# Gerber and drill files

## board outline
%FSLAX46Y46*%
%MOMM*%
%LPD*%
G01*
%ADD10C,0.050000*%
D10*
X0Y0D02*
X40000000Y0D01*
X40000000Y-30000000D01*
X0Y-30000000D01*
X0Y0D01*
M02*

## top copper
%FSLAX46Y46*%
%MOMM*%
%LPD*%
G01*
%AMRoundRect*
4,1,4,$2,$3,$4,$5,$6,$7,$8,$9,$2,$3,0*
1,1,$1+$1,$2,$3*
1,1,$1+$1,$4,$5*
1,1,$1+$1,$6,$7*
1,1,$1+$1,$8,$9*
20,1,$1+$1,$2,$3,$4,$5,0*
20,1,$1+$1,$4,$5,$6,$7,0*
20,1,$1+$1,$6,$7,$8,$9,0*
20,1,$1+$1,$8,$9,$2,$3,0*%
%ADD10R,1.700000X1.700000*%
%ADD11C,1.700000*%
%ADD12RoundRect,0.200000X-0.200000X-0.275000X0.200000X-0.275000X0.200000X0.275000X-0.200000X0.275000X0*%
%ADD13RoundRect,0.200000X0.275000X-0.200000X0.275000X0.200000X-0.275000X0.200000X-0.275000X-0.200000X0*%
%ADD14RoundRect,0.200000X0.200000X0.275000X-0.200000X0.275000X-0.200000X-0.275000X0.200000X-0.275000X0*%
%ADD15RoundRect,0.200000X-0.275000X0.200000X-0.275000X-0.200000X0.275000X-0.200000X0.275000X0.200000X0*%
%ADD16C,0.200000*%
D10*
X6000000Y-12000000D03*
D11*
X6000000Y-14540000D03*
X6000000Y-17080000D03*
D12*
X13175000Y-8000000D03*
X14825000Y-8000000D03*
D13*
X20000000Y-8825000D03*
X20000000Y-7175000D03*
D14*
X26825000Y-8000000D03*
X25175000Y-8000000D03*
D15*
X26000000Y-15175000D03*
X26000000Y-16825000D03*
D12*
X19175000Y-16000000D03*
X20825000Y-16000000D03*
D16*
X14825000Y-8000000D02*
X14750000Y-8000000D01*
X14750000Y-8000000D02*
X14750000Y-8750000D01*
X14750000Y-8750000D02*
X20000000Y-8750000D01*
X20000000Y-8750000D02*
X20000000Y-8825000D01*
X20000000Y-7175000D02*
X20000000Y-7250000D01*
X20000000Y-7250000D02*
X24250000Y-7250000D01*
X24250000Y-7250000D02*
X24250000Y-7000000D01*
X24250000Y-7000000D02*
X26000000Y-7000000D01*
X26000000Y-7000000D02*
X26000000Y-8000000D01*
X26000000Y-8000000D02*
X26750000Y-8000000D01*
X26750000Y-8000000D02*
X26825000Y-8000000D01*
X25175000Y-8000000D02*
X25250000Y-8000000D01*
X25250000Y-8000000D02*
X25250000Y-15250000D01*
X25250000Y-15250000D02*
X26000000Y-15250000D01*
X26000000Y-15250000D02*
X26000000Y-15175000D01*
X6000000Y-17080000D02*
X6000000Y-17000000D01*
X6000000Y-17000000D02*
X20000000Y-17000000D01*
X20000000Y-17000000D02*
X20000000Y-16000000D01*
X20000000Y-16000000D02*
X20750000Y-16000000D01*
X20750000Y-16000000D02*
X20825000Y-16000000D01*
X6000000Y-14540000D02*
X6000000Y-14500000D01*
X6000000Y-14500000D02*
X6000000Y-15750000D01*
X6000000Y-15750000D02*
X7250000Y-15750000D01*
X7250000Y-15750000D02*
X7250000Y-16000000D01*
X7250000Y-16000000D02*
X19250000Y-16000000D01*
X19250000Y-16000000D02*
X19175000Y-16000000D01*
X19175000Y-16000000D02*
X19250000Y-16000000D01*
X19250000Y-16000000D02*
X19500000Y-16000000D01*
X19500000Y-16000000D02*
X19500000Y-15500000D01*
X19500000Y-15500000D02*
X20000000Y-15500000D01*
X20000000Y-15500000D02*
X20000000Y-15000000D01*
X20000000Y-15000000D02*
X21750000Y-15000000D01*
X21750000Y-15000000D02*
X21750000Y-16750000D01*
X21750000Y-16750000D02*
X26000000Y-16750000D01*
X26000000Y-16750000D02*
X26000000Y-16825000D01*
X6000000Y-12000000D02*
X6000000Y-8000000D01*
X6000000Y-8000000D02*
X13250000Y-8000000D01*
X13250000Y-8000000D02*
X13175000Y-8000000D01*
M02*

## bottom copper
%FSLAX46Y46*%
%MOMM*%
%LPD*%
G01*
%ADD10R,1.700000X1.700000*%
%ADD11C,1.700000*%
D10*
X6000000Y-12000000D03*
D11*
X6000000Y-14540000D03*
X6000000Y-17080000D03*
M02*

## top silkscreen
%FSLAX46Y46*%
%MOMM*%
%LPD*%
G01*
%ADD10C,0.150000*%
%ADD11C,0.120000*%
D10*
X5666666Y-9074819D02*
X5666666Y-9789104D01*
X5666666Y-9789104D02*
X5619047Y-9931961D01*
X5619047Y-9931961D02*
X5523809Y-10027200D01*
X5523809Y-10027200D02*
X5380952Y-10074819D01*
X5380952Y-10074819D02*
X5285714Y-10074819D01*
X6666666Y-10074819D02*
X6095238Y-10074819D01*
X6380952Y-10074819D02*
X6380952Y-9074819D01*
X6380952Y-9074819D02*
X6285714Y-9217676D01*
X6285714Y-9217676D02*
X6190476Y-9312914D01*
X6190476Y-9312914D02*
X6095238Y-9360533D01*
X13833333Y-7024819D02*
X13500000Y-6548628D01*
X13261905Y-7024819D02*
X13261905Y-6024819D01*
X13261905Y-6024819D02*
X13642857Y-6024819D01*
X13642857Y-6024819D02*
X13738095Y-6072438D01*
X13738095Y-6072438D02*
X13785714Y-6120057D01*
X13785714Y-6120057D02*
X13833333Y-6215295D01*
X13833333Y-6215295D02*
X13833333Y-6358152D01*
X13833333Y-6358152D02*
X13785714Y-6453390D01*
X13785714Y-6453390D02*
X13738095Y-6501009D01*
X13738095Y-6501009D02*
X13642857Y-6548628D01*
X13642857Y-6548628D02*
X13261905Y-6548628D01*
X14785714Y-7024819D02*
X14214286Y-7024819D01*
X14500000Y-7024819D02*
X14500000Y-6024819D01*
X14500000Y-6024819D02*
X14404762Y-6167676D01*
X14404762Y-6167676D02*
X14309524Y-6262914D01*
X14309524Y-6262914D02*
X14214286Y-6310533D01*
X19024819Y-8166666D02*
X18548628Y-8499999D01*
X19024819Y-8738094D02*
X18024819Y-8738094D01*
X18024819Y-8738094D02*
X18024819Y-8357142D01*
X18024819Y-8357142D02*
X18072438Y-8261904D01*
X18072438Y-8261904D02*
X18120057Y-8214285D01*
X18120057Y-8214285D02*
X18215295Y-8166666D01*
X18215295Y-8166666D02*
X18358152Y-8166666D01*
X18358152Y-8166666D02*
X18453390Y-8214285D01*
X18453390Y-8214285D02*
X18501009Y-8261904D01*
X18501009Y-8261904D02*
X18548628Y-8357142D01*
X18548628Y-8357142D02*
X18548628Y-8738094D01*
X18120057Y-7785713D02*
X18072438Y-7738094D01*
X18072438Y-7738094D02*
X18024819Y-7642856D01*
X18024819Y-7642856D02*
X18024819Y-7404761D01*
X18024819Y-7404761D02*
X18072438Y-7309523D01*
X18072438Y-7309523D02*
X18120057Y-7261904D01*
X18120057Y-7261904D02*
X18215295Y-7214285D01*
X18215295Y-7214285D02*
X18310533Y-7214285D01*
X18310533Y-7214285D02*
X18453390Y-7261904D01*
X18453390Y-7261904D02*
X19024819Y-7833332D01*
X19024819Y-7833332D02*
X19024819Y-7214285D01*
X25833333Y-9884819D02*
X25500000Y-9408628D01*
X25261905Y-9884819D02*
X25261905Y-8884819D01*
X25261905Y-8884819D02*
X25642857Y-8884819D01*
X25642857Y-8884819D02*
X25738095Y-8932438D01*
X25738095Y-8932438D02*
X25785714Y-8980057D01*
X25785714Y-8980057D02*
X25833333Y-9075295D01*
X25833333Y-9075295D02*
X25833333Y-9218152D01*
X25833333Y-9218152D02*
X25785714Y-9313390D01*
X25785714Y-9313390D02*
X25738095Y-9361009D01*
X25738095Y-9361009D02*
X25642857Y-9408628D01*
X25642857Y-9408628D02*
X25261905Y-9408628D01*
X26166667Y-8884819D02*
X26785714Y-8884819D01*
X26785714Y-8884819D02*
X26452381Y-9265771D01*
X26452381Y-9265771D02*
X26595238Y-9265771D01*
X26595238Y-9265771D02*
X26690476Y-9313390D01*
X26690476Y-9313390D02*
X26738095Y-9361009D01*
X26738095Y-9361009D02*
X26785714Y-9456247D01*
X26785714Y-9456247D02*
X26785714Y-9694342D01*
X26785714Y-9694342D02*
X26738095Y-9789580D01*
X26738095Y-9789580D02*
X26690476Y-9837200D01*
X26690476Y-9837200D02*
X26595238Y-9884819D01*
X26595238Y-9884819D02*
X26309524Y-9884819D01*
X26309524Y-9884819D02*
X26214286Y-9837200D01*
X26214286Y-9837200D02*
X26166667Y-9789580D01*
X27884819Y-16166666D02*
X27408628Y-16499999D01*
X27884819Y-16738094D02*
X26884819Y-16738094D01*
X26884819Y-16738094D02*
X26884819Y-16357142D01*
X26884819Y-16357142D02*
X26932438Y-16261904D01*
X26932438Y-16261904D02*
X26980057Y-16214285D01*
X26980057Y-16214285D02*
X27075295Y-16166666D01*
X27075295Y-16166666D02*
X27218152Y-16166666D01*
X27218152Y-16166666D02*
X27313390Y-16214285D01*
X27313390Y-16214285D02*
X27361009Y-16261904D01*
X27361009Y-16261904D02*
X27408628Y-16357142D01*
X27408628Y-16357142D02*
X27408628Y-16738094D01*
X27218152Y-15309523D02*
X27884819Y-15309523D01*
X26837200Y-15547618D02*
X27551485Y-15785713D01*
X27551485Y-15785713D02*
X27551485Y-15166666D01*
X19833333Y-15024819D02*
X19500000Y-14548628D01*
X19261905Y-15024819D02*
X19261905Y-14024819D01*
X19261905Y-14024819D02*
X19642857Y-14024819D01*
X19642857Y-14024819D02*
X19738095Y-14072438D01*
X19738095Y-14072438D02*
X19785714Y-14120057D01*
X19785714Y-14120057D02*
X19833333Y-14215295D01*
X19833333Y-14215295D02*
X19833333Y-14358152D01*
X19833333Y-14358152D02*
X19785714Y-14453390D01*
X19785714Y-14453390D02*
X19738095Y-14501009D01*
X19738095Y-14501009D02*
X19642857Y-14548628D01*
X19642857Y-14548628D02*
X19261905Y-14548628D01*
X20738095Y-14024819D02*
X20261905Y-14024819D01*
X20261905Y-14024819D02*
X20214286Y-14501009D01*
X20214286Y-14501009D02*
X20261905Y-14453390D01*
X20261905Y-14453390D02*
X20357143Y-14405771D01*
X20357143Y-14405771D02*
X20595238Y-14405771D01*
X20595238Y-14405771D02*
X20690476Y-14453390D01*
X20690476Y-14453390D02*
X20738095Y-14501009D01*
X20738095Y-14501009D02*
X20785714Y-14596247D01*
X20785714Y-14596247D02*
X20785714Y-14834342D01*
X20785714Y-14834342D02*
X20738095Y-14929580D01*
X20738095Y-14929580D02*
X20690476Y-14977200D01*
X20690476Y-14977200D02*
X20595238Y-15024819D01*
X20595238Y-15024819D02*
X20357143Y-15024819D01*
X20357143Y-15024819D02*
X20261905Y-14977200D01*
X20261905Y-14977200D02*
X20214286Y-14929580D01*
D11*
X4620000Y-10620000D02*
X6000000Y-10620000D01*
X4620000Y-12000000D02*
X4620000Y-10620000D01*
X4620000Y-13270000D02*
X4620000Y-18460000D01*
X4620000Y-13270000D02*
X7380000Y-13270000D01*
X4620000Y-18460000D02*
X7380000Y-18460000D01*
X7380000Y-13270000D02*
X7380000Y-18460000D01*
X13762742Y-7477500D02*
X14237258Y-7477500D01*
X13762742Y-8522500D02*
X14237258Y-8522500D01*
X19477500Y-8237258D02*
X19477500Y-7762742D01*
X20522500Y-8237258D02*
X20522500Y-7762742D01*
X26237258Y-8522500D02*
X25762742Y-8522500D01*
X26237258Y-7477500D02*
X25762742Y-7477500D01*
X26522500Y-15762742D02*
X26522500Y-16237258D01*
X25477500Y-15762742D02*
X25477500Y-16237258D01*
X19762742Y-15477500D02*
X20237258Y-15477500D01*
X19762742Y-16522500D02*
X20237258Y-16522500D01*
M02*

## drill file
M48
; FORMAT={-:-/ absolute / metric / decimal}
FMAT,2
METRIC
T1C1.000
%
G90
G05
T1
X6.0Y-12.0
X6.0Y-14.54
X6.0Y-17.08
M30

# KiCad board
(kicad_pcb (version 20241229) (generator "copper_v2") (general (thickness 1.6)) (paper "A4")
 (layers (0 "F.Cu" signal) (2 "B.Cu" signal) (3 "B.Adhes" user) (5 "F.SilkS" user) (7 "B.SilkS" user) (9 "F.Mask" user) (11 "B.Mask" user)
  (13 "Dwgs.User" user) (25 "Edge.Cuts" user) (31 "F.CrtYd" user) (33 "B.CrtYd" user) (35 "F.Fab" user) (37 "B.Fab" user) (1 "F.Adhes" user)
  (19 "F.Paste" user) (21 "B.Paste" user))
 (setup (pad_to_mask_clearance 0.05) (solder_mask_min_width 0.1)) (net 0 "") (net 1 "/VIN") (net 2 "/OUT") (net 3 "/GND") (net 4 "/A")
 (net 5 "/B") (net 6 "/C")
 (gr_rect (start 0 0) (end 40 30) (stroke (width .05) (type default)) (fill none) (layer "Edge.Cuts"))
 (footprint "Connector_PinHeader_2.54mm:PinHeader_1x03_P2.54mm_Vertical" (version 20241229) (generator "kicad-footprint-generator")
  (layer "F.Cu")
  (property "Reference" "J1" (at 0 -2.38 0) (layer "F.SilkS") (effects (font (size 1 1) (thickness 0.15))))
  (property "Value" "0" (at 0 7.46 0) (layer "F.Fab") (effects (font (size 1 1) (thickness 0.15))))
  (fp_line (start -1.38 -1.38) (end 0 -1.38) (stroke (width 0.12) (type solid)) (layer "F.SilkS"))
  (fp_line (start -1.38 0) (end -1.38 -1.38) (stroke (width 0.12) (type solid)) (layer "F.SilkS"))
  (fp_line (start -1.38 1.27) (end -1.38 6.46) (stroke (width 0.12) (type solid)) (layer "F.SilkS"))
  (fp_line (start -1.38 1.27) (end 1.38 1.27) (stroke (width 0.12) (type solid)) (layer "F.SilkS"))
  (fp_line (start -1.38 6.46) (end 1.38 6.46) (stroke (width 0.12) (type solid)) (layer "F.SilkS"))
  (fp_line (start 1.38 1.27) (end 1.38 6.46) (stroke (width 0.12) (type solid)) (layer "F.SilkS"))
  (pad "1" thru_hole rect (at 0 0) (size 1.7 1.7) (drill 1) (layers "*.Cu" "*.Mask") (remove_unused_layers no) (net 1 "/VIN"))
  (pad "2" thru_hole circle (at 0 2.54) (size 1.7 1.7) (drill 1) (layers "*.Cu" "*.Mask") (remove_unused_layers no) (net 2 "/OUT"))
  (pad "3" thru_hole circle (at 0 5.08) (size 1.7 1.7) (drill 1) (layers "*.Cu" "*.Mask") (remove_unused_layers no) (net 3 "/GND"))
  (at 6 12 0))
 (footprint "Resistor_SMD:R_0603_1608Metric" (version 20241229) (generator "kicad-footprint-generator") (layer "F.Cu")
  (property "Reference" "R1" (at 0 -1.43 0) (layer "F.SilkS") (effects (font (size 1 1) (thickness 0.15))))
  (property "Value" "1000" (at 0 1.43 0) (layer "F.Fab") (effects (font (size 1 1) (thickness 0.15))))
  (fp_line (start -0.237258 -0.5225) (end 0.237258 -0.5225) (stroke (width 0.12) (type solid)) (layer "F.SilkS"))
  (fp_line (start -0.237258 0.5225) (end 0.237258 0.5225) (stroke (width 0.12) (type solid)) (layer "F.SilkS"))
  (pad "1" smd roundrect (at -0.825 0) (size 0.8 0.95) (layers "F.Cu" "F.Mask" "F.Paste") (roundrect_rratio 0.25) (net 1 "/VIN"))
  (pad "2" smd roundrect (at 0.825 0) (size 0.8 0.95) (layers "F.Cu" "F.Mask" "F.Paste") (roundrect_rratio 0.25) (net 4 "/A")) (at 14 8 0))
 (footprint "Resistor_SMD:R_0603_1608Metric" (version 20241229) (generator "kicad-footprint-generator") (layer "F.Cu")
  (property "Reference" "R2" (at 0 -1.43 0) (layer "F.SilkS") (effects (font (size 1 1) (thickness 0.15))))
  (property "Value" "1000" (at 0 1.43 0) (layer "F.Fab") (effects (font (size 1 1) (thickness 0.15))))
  (fp_line (start -0.237258 -0.5225) (end 0.237258 -0.5225) (stroke (width 0.12) (type solid)) (layer "F.SilkS"))
  (fp_line (start -0.237258 0.5225) (end 0.237258 0.5225) (stroke (width 0.12) (type solid)) (layer "F.SilkS"))
  (pad "1" smd roundrect (at -0.825 0) (size 0.8 0.95) (layers "F.Cu" "F.Mask" "F.Paste") (roundrect_rratio 0.25) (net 4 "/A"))
  (pad "2" smd roundrect (at 0.825 0) (size 0.8 0.95) (layers "F.Cu" "F.Mask" "F.Paste") (roundrect_rratio 0.25) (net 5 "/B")) (at 20 8 90))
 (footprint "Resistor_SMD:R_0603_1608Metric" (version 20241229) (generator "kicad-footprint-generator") (layer "F.Cu")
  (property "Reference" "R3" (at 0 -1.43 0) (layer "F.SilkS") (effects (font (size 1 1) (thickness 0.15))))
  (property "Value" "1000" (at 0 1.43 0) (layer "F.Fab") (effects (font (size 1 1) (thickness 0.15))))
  (fp_line (start -0.237258 -0.5225) (end 0.237258 -0.5225) (stroke (width 0.12) (type solid)) (layer "F.SilkS"))
  (fp_line (start -0.237258 0.5225) (end 0.237258 0.5225) (stroke (width 0.12) (type solid)) (layer "F.SilkS"))
  (pad "1" smd roundrect (at -0.825 0) (size 0.8 0.95) (layers "F.Cu" "F.Mask" "F.Paste") (roundrect_rratio 0.25) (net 5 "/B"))
  (pad "2" smd roundrect (at 0.825 0) (size 0.8 0.95) (layers "F.Cu" "F.Mask" "F.Paste") (roundrect_rratio 0.25) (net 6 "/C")) (at 26 8 180))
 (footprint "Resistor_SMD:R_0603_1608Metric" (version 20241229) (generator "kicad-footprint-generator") (layer "F.Cu")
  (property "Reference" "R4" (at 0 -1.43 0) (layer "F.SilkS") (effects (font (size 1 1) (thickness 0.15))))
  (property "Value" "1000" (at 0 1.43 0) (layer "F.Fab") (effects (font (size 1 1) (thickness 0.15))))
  (fp_line (start -0.237258 -0.5225) (end 0.237258 -0.5225) (stroke (width 0.12) (type solid)) (layer "F.SilkS"))
  (fp_line (start -0.237258 0.5225) (end 0.237258 0.5225) (stroke (width 0.12) (type solid)) (layer "F.SilkS"))
  (pad "1" smd roundrect (at -0.825 0) (size 0.8 0.95) (layers "F.Cu" "F.Mask" "F.Paste") (roundrect_rratio 0.25) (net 6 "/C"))
  (pad "2" smd roundrect (at 0.825 0) (size 0.8 0.95) (layers "F.Cu" "F.Mask" "F.Paste") (roundrect_rratio 0.25) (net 2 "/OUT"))
  (at 26 16 270))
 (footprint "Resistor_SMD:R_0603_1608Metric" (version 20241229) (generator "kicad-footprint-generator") (layer "F.Cu")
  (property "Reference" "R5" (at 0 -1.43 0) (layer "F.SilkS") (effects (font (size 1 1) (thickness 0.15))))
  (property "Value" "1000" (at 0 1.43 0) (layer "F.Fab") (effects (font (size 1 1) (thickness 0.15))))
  (fp_line (start -0.237258 -0.5225) (end 0.237258 -0.5225) (stroke (width 0.12) (type solid)) (layer "F.SilkS"))
  (fp_line (start -0.237258 0.5225) (end 0.237258 0.5225) (stroke (width 0.12) (type solid)) (layer "F.SilkS"))
  (pad "1" smd roundrect (at -0.825 0) (size 0.8 0.95) (layers "F.Cu" "F.Mask" "F.Paste") (roundrect_rratio 0.25) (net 2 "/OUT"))
  (pad "2" smd roundrect (at 0.825 0) (size 0.8 0.95) (layers "F.Cu" "F.Mask" "F.Paste") (roundrect_rratio 0.25) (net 3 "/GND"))
  (at 20 16 0))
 (segment (start 14.825 8) (end 14.75 8) (width 0.2) (layer "F.Cu") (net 4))
 (segment (start 14.75 8) (end 14.75 8.75) (width 0.2) (layer "F.Cu") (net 4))
 (segment (start 14.75 8.75) (end 20 8.75) (width 0.2) (layer "F.Cu") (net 4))
 (segment (start 20 8.75) (end 20 8.825) (width 0.2) (layer "F.Cu") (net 4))
 (segment (start 20 7.175) (end 20 7.25) (width 0.2) (layer "F.Cu") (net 5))
 (segment (start 20 7.25) (end 24.25 7.25) (width 0.2) (layer "F.Cu") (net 5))
 (segment (start 24.25 7.25) (end 24.25 7) (width 0.2) (layer "F.Cu") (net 5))
 (segment (start 24.25 7) (end 26 7) (width 0.2) (layer "F.Cu") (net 5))
 (segment (start 26 7) (end 26 8) (width 0.2) (layer "F.Cu") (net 5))
 (segment (start 26 8) (end 26.75 8) (width 0.2) (layer "F.Cu") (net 5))
 (segment (start 26.75 8) (end 26.825 8) (width 0.2) (layer "F.Cu") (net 5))
 (segment (start 25.175 8) (end 25.25 8) (width 0.2) (layer "F.Cu") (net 6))
 (segment (start 25.25 8) (end 25.25 15.25) (width 0.2) (layer "F.Cu") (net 6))
 (segment (start 25.25 15.25) (end 26 15.25) (width 0.2) (layer "F.Cu") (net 6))
 (segment (start 26 15.25) (end 26 15.175) (width 0.2) (layer "F.Cu") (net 6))
 (segment (start 6 17.08) (end 6 17) (width 0.2) (layer "F.Cu") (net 3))
 (segment (start 6 17) (end 20 17) (width 0.2) (layer "F.Cu") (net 3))
 (segment (start 20 17) (end 20 16) (width 0.2) (layer "F.Cu") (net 3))
 (segment (start 20 16) (end 20.75 16) (width 0.2) (layer "F.Cu") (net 3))
 (segment (start 20.75 16) (end 20.825 16) (width 0.2) (layer "F.Cu") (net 3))
 (segment (start 6 14.54) (end 6 14.5) (width 0.2) (layer "F.Cu") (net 2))
 (segment (start 6 14.5) (end 6 15.75) (width 0.2) (layer "F.Cu") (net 2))
 (segment (start 6 15.75) (end 7.25 15.75) (width 0.2) (layer "F.Cu") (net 2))
 (segment (start 7.25 15.75) (end 7.25 16) (width 0.2) (layer "F.Cu") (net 2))
 (segment (start 7.25 16) (end 19.25 16) (width 0.2) (layer "F.Cu") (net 2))
 (segment (start 19.25 16) (end 19.175 16) (width 0.2) (layer "F.Cu") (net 2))
 (segment (start 19.175 16) (end 19.25 16) (width 0.2) (layer "F.Cu") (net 2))
 (segment (start 19.25 16) (end 19.5 16) (width 0.2) (layer "F.Cu") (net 2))
 (segment (start 19.5 16) (end 19.5 15.5) (width 0.2) (layer "F.Cu") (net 2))
 (segment (start 19.5 15.5) (end 20 15.5) (width 0.2) (layer "F.Cu") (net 2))
 (segment (start 20 15.5) (end 20 15) (width 0.2) (layer "F.Cu") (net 2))
 (segment (start 20 15) (end 21.75 15) (width 0.2) (layer "F.Cu") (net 2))
 (segment (start 21.75 15) (end 21.75 16.75) (width 0.2) (layer "F.Cu") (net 2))
 (segment (start 21.75 16.75) (end 26 16.75) (width 0.2) (layer "F.Cu") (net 2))
 (segment (start 26 16.75) (end 26 16.825) (width 0.2) (layer "F.Cu") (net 2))
 (segment (start 6 12) (end 6 8) (width 0.2) (layer "F.Cu") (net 1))
 (segment (start 6 8) (end 13.25 8) (width 0.2) (layer "F.Cu") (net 1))
 (segment (start 13.25 8) (end 13.175 8) (width 0.2) (layer "F.Cu") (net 1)))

